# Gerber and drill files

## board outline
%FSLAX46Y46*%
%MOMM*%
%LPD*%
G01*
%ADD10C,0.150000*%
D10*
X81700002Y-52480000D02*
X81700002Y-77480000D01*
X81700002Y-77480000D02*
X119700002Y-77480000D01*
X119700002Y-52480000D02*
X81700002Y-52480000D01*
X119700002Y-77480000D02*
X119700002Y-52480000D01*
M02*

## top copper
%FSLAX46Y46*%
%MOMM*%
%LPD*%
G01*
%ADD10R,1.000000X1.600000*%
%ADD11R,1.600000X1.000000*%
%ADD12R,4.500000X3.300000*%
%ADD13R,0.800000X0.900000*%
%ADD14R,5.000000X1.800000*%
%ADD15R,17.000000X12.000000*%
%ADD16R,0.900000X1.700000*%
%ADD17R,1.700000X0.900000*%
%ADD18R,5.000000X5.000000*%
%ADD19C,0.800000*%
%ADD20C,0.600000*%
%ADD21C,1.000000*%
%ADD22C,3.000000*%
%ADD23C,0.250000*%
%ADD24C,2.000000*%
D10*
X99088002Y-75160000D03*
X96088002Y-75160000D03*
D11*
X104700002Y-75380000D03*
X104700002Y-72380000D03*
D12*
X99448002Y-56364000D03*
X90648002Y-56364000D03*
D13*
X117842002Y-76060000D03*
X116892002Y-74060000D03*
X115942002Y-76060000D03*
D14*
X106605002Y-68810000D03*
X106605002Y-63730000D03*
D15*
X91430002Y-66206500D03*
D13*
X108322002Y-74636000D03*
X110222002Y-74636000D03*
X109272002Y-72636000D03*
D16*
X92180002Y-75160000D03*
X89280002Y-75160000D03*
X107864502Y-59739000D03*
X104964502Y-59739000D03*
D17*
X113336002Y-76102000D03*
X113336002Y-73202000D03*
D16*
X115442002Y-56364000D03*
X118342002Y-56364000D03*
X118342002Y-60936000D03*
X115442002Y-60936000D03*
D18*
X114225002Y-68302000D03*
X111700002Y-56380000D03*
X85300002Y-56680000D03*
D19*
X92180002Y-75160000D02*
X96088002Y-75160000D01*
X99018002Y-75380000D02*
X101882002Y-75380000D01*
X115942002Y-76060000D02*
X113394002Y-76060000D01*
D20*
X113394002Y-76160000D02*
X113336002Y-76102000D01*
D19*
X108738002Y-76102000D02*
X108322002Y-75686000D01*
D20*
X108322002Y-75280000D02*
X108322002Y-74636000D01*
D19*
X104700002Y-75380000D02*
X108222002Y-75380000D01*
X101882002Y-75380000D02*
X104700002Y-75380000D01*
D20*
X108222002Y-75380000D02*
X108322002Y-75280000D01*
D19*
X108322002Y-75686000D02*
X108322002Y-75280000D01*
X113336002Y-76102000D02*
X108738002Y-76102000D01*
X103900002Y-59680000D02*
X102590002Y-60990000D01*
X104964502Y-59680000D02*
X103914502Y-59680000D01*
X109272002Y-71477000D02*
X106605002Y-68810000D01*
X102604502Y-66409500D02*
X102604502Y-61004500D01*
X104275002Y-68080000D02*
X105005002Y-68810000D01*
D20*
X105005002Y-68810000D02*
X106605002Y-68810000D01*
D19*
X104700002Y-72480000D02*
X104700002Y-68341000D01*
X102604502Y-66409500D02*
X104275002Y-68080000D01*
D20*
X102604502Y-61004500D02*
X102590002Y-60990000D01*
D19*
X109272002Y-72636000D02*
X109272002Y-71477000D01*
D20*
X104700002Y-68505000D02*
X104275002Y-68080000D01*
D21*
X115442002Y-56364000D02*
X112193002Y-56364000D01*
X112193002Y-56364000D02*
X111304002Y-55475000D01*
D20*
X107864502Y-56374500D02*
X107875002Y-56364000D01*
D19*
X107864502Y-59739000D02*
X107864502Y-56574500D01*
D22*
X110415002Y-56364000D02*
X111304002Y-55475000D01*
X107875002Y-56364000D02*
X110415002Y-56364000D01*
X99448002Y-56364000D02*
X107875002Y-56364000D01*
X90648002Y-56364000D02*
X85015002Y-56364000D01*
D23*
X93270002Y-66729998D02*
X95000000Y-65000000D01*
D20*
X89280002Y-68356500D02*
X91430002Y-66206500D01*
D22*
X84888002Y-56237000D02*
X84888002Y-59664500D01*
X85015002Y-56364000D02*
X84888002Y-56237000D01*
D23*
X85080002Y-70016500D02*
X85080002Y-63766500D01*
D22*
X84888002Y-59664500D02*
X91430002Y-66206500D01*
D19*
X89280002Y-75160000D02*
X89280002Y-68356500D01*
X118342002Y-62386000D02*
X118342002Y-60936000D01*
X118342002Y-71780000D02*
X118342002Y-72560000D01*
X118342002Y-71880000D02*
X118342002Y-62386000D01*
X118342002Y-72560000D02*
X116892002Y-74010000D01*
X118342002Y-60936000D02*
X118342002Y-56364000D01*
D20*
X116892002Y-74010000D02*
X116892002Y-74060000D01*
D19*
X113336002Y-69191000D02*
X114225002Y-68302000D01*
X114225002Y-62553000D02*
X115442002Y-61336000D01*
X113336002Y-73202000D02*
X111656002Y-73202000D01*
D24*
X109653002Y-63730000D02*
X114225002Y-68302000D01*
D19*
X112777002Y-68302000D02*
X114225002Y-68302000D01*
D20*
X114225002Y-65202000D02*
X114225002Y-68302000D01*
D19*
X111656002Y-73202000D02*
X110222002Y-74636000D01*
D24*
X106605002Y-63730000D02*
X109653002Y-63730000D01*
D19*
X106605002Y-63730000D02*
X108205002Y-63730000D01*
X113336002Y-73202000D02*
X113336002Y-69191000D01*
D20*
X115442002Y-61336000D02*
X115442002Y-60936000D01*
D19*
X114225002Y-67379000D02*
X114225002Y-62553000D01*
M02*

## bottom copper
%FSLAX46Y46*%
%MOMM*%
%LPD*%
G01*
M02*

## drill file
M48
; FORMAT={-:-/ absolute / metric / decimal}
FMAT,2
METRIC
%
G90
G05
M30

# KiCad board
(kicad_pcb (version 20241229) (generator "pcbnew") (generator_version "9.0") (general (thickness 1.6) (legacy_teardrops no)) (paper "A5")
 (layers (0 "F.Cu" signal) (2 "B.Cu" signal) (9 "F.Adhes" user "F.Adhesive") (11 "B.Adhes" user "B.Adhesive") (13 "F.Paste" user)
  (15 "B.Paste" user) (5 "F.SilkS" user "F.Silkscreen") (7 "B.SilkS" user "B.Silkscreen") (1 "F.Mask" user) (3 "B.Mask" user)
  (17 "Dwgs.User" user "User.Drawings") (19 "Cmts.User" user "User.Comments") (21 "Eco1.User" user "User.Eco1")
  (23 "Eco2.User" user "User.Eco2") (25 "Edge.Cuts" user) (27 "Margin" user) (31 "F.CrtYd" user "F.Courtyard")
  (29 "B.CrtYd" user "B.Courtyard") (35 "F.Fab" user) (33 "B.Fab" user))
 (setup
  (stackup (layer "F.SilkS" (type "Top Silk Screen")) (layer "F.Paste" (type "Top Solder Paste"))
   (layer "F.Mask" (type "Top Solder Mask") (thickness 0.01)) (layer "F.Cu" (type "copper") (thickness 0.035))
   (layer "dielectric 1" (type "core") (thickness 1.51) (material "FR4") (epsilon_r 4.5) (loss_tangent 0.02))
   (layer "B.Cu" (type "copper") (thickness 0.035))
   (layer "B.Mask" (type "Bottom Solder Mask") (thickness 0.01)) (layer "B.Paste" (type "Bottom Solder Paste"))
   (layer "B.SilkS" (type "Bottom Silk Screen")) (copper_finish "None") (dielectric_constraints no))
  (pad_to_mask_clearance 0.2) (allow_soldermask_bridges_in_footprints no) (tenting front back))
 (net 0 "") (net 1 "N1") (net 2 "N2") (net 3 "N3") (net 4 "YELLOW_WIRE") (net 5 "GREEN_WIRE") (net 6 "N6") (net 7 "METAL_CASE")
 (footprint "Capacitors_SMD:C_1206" (layer "F.Cu") (at 97.588002 75.16 180)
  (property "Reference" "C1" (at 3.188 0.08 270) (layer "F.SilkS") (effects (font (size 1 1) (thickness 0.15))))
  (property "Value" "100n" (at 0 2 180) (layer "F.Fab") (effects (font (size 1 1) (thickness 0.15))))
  (pad "1" smd rect (at -1.5 0 180) (size 1 1.6) (layers "F.Cu" "F.Mask" "F.Paste") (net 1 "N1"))
  (pad "2" smd rect (at 1.5 0 180) (size 1 1.6) (layers "F.Cu" "F.Mask" "F.Paste") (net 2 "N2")))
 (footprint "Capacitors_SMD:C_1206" (layer "F.Cu") (at 104.700002 73.88 90)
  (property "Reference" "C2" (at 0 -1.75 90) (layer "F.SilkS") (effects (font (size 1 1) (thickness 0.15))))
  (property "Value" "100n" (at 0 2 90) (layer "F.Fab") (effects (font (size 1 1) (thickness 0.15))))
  (pad "1" smd rect (at -1.5 0 90) (size 1 1.6) (layers "F.Cu" "F.Mask" "F.Paste") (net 1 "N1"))
  (pad "2" smd rect (at 1.5 0 90) (size 1 1.6) (layers "F.Cu" "F.Mask" "F.Paste") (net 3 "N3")))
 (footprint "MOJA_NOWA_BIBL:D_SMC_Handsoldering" (layer "F.Cu") (at 95.048002 56.364 180)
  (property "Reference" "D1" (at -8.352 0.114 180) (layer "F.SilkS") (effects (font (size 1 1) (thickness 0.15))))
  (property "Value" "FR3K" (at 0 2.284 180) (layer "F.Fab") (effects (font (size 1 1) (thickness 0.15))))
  (pad "1" smd rect (at -4.4 0 270) (size 3.3 4.5) (layers "F.Cu" "F.Mask" "F.Paste") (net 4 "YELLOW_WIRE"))
  (pad "2" smd rect (at 4.4 0 270) (size 3.3 4.5) (layers "F.Cu" "F.Mask" "F.Paste") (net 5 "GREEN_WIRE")))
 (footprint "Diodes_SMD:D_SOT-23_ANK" (layer "F.Cu") (at 116.892002 75.06 90)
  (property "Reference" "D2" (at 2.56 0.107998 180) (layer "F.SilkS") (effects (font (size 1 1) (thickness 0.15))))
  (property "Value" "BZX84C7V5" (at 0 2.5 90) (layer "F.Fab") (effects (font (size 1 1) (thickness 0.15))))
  (pad "" smd rect (at -1 0.95 90) (size 0.9 0.8) (layers "F.Cu" "F.Mask" "F.Paste"))
  (pad "1" smd rect (at 1 0 90) (size 0.9 0.8) (layers "F.Cu" "F.Mask" "F.Paste") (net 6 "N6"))
  (pad "2" smd rect (at -1 -0.95 90) (size 0.9 0.8) (layers "F.Cu" "F.Mask" "F.Paste") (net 1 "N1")))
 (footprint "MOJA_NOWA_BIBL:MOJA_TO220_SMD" (layer "F.Cu") (at 103.430002 68.81 90)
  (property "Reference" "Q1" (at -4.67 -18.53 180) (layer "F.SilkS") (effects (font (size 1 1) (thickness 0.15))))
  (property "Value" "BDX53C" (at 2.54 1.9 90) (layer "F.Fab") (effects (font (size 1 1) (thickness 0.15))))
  (pad "1" smd rect (at 0 3.175 90) (size 1.8 5) (layers "F.Cu" "F.Mask" "F.Paste") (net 3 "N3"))
  (pad "2" smd rect (at 5.08 3.175 90) (size 1.8 5) (layers "F.Cu" "F.Mask" "F.Paste") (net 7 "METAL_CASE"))
  (pad "3" smd rect (at 2.6035 -12 90) (size 12 17) (layers "F.Cu" "F.Mask" "F.Paste") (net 5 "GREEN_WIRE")))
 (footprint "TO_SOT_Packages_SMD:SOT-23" (layer "F.Cu") (at 109.272002 73.636 90)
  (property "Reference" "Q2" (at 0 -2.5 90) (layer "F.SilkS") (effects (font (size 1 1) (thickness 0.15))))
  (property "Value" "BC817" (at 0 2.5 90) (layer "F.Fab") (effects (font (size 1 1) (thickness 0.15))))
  (pad "1" smd rect (at -1 -0.95 90) (size 0.9 0.8) (layers "F.Cu" "F.Mask" "F.Paste") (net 1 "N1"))
  (pad "2" smd rect (at -1 0.95 90) (size 0.9 0.8) (layers "F.Cu" "F.Mask" "F.Paste") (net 7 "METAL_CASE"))
  (pad "3" smd rect (at 1 0 90) (size 0.9 0.8) (layers "F.Cu" "F.Mask" "F.Paste") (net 3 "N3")))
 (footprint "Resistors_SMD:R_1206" (layer "F.Cu") (at 90.730002 75.16 180)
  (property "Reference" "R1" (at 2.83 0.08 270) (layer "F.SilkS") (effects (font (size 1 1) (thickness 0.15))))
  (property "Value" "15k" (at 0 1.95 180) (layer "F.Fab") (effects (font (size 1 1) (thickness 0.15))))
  (pad "1" smd rect (at -1.45 0 180) (size 0.9 1.7) (layers "F.Cu" "F.Mask" "F.Paste") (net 2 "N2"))
  (pad "2" smd rect (at 1.45 0 180) (size 0.9 1.7) (layers "F.Cu" "F.Mask" "F.Paste") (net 5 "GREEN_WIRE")))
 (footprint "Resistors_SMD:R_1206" (layer "F.Cu") (at 106.414502 59.739 180)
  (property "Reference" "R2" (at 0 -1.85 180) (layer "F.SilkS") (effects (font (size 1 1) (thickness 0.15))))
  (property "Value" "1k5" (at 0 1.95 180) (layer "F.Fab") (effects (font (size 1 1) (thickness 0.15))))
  (pad "1" smd rect (at -1.45 0 180) (size 0.9 1.7) (layers "F.Cu" "F.Mask" "F.Paste") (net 4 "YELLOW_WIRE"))
  (pad "2" smd rect (at 1.45 0 180) (size 0.9 1.7) (layers "F.Cu" "F.Mask" "F.Paste") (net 3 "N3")))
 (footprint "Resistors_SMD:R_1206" (layer "F.Cu") (at 113.336002 74.652 90)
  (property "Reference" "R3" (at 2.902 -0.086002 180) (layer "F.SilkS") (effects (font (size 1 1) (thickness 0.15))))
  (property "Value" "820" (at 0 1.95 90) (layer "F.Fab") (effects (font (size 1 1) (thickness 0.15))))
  (pad "1" smd rect (at -1.45 0 90) (size 0.9 1.7) (layers "F.Cu" "F.Mask" "F.Paste") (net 1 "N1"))
  (pad "2" smd rect (at 1.45 0 90) (size 0.9 1.7) (layers "F.Cu" "F.Mask" "F.Paste") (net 7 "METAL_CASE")))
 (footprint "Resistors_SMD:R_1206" (layer "F.Cu") (at 116.892002 56.364)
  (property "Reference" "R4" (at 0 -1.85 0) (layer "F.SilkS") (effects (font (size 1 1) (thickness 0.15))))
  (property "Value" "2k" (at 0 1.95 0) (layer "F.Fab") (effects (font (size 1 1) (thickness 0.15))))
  (pad "1" smd rect (at -1.45 0) (size 0.9 1.7) (layers "F.Cu" "F.Mask" "F.Paste") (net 4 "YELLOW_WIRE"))
  (pad "2" smd rect (at 1.45 0) (size 0.9 1.7) (layers "F.Cu" "F.Mask" "F.Paste") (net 6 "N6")))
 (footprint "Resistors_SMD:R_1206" (layer "F.Cu") (at 116.892002 60.936 180)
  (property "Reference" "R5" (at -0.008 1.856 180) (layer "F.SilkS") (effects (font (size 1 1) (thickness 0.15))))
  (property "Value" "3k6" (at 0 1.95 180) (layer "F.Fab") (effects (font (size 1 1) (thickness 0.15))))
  (pad "1" smd rect (at -1.45 0 180) (size 0.9 1.7) (layers "F.Cu" "F.Mask" "F.Paste") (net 6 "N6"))
  (pad "2" smd rect (at 1.45 0 180) (size 0.9 1.7) (layers "F.Cu" "F.Mask" "F.Paste") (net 7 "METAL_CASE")))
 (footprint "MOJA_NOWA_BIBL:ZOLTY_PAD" (layer "F.Cu") (at 114.352002 64.746)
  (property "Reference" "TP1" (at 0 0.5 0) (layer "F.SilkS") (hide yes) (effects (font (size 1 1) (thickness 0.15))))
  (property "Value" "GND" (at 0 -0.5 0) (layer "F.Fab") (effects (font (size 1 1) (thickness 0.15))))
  (pad "1" smd rect (at -0.127 3.556) (size 5 5) (layers "F.Cu" "F.Mask" "F.Paste") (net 7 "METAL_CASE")))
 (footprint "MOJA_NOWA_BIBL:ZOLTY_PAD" (layer "F.Cu") (at 108.144002 56.253 90)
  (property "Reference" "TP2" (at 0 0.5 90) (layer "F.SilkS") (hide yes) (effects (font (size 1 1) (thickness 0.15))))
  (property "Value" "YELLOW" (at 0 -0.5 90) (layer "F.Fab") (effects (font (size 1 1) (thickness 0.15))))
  (pad "1" smd rect (at -0.127 3.556 90) (size 5 5) (layers "F.Cu" "F.Mask" "F.Paste") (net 4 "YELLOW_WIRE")))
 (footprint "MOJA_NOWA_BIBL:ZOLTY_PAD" (layer "F.Cu") (at 88.856002 56.807 -90)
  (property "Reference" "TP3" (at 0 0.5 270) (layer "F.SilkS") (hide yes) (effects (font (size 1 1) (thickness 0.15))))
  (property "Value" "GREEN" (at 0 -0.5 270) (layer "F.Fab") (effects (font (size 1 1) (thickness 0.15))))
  (pad "1" smd rect (at -0.127 3.556 270) (size 5 5) (layers "F.Cu" "F.Mask" "F.Paste") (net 5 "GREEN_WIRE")))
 (gr_line (start 81.700002 52.48) (end 81.700002 77.48) (stroke (width 0.15) (type solid)) (layer "Edge.Cuts"))
 (gr_line (start 81.700002 77.48) (end 119.700002 77.48) (stroke (width 0.15) (type solid)) (layer "Edge.Cuts"))
 (gr_line (start 119.700002 52.48) (end 81.700002 52.48) (stroke (width 0.15) (type solid)) (layer "Edge.Cuts"))
 (gr_line (start 119.700002 77.48) (end 119.700002 52.48) (stroke (width 0.15) (type solid)) (layer "Edge.Cuts"))
 (segment (start 92.180002 75.16) (end 96.088002 75.16) (width 0.8) (layer "F.Cu") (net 2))
 (segment (start 99.018002 75.38) (end 101.882002 75.38) (width 0.8) (layer "F.Cu") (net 1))
 (segment (start 115.942002 76.06) (end 113.394002 76.06) (width 0.8) (layer "F.Cu") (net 1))
 (segment (start 113.394002 76.16) (end 113.336002 76.102) (width 0.6) (layer "F.Cu") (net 1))
 (segment (start 108.738002 76.102) (end 108.322002 75.686) (width 0.8) (layer "F.Cu") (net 1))
 (segment (start 108.322002 75.28) (end 108.322002 74.636) (width 0.6) (layer "F.Cu") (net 1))
 (segment (start 104.700002 75.38) (end 108.222002 75.38) (width 0.8) (layer "F.Cu") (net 1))
 (segment (start 101.882002 75.38) (end 104.700002 75.38) (width 0.8) (layer "F.Cu") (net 1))
 (segment (start 108.222002 75.38) (end 108.322002 75.28) (width 0.6) (layer "F.Cu") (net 1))
 (segment (start 108.322002 75.686) (end 108.322002 75.28) (width 0.8) (layer "F.Cu") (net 1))
 (segment (start 113.336002 76.102) (end 108.738002 76.102) (width 0.8) (layer "F.Cu") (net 1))
 (segment (start 103.900002 59.68) (end 102.590002 60.99) (width 0.8) (layer "F.Cu") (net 3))
 (segment (start 104.964502 59.68) (end 103.914502 59.68) (width 0.8) (layer "F.Cu") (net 3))
 (segment (start 109.272002 71.477) (end 106.605002 68.81) (width 0.8) (layer "F.Cu") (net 3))
 (segment (start 102.604502 66.4095) (end 102.604502 61.0045) (width 0.8) (layer "F.Cu") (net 3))
 (segment (start 104.275002 68.08) (end 105.005002 68.81) (width 0.8) (layer "F.Cu") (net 3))
 (segment (start 105.005002 68.81) (end 106.605002 68.81) (width 0.6) (layer "F.Cu") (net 3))
 (segment (start 104.700002 72.48) (end 104.700002 68.341) (width 0.8) (layer "F.Cu") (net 3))
 (segment (start 102.604502 66.4095) (end 104.275002 68.08) (width 0.8) (layer "F.Cu") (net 3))
 (segment (start 102.604502 61.0045) (end 102.590002 60.99) (width 0.6) (layer "F.Cu") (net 3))
 (segment (start 109.272002 72.636) (end 109.272002 71.477) (width 0.8) (layer "F.Cu") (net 3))
 (segment (start 104.700002 68.505) (end 104.275002 68.08) (width 0.6) (layer "F.Cu") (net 3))
 (segment (start 115.442002 56.364) (end 112.193002 56.364) (width 1) (layer "F.Cu") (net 4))
 (segment (start 112.193002 56.364) (end 111.304002 55.475) (width 1) (layer "F.Cu") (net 4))
 (segment (start 107.864502 56.3745) (end 107.875002 56.364) (width 0.6) (layer "F.Cu") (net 4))
 (segment (start 107.864502 59.739) (end 107.864502 56.5745) (width 0.8) (layer "F.Cu") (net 4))
 (segment (start 110.415002 56.364) (end 111.304002 55.475) (width 3) (layer "F.Cu") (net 4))
 (segment (start 107.875002 56.364) (end 110.415002 56.364) (width 3) (layer "F.Cu") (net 4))
 (segment (start 99.448002 56.364) (end 107.875002 56.364) (width 3) (layer "F.Cu") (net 4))
 (segment (start 90.648002 56.364) (end 85.015002 56.364) (width 3) (layer "F.Cu") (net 5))
 (segment (start 93.270002 66.729998) (end 95 65) (width 0.25) (layer "F.Cu") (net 5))
 (segment (start 89.280002 68.3565) (end 91.430002 66.2065) (width 0.6) (layer "F.Cu") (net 5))
 (segment (start 84.888002 56.237) (end 84.888002 59.6645) (width 3) (layer "F.Cu") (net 5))
 (segment (start 85.015002 56.364) (end 84.888002 56.237) (width 3) (layer "F.Cu") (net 5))
 (segment (start 85.080002 70.0165) (end 85.080002 63.7665) (width 0.25) (layer "F.Cu") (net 5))
 (segment (start 84.888002 59.6645) (end 91.430002 66.2065) (width 3) (layer "F.Cu") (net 5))
 (segment (start 89.280002 75.16) (end 89.280002 68.3565) (width 0.8) (layer "F.Cu") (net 5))
 (segment (start 118.342002 62.386) (end 118.342002 60.936) (width 0.8) (layer "F.Cu") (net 6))
 (segment (start 118.342002 71.78) (end 118.342002 72.56) (width 0.8) (layer "F.Cu") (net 6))
 (segment (start 118.342002 71.88) (end 118.342002 62.386) (width 0.8) (layer "F.Cu") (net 6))
 (segment (start 118.342002 72.56) (end 116.892002 74.01) (width 0.8) (layer "F.Cu") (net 6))
 (segment (start 118.342002 60.936) (end 118.342002 56.364) (width 0.8) (layer "F.Cu") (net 6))
 (segment (start 116.892002 74.01) (end 116.892002 74.06) (width 0.6) (layer "F.Cu") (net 6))
 (segment (start 113.336002 69.191) (end 114.225002 68.302) (width 0.8) (layer "F.Cu") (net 7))
 (segment (start 114.225002 62.553) (end 115.442002 61.336) (width 0.8) (layer "F.Cu") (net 7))
 (segment (start 113.336002 73.202) (end 111.656002 73.202) (width 0.8) (layer "F.Cu") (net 7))
 (segment (start 109.653002 63.73) (end 114.225002 68.302) (width 2) (layer "F.Cu") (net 7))
 (segment (start 112.777002 68.302) (end 114.225002 68.302) (width 0.8) (layer "F.Cu") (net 7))
 (segment (start 114.225002 65.202) (end 114.225002 68.302) (width 0.6) (layer "F.Cu") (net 7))
 (segment (start 111.656002 73.202) (end 110.222002 74.636) (width 0.8) (layer "F.Cu") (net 7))
 (segment (start 106.605002 63.73) (end 109.653002 63.73) (width 2) (layer "F.Cu") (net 7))
 (segment (start 106.605002 63.73) (end 108.205002 63.73) (width 0.8) (layer "F.Cu") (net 7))
 (segment (start 113.336002 73.202) (end 113.336002 69.191) (width 0.8) (layer "F.Cu") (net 7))
 (segment (start 115.442002 61.336) (end 115.442002 60.936) (width 0.6) (layer "F.Cu") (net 7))
 (segment (start 114.225002 67.379) (end 114.225002 62.553) (width 0.8) (layer "F.Cu") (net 7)))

